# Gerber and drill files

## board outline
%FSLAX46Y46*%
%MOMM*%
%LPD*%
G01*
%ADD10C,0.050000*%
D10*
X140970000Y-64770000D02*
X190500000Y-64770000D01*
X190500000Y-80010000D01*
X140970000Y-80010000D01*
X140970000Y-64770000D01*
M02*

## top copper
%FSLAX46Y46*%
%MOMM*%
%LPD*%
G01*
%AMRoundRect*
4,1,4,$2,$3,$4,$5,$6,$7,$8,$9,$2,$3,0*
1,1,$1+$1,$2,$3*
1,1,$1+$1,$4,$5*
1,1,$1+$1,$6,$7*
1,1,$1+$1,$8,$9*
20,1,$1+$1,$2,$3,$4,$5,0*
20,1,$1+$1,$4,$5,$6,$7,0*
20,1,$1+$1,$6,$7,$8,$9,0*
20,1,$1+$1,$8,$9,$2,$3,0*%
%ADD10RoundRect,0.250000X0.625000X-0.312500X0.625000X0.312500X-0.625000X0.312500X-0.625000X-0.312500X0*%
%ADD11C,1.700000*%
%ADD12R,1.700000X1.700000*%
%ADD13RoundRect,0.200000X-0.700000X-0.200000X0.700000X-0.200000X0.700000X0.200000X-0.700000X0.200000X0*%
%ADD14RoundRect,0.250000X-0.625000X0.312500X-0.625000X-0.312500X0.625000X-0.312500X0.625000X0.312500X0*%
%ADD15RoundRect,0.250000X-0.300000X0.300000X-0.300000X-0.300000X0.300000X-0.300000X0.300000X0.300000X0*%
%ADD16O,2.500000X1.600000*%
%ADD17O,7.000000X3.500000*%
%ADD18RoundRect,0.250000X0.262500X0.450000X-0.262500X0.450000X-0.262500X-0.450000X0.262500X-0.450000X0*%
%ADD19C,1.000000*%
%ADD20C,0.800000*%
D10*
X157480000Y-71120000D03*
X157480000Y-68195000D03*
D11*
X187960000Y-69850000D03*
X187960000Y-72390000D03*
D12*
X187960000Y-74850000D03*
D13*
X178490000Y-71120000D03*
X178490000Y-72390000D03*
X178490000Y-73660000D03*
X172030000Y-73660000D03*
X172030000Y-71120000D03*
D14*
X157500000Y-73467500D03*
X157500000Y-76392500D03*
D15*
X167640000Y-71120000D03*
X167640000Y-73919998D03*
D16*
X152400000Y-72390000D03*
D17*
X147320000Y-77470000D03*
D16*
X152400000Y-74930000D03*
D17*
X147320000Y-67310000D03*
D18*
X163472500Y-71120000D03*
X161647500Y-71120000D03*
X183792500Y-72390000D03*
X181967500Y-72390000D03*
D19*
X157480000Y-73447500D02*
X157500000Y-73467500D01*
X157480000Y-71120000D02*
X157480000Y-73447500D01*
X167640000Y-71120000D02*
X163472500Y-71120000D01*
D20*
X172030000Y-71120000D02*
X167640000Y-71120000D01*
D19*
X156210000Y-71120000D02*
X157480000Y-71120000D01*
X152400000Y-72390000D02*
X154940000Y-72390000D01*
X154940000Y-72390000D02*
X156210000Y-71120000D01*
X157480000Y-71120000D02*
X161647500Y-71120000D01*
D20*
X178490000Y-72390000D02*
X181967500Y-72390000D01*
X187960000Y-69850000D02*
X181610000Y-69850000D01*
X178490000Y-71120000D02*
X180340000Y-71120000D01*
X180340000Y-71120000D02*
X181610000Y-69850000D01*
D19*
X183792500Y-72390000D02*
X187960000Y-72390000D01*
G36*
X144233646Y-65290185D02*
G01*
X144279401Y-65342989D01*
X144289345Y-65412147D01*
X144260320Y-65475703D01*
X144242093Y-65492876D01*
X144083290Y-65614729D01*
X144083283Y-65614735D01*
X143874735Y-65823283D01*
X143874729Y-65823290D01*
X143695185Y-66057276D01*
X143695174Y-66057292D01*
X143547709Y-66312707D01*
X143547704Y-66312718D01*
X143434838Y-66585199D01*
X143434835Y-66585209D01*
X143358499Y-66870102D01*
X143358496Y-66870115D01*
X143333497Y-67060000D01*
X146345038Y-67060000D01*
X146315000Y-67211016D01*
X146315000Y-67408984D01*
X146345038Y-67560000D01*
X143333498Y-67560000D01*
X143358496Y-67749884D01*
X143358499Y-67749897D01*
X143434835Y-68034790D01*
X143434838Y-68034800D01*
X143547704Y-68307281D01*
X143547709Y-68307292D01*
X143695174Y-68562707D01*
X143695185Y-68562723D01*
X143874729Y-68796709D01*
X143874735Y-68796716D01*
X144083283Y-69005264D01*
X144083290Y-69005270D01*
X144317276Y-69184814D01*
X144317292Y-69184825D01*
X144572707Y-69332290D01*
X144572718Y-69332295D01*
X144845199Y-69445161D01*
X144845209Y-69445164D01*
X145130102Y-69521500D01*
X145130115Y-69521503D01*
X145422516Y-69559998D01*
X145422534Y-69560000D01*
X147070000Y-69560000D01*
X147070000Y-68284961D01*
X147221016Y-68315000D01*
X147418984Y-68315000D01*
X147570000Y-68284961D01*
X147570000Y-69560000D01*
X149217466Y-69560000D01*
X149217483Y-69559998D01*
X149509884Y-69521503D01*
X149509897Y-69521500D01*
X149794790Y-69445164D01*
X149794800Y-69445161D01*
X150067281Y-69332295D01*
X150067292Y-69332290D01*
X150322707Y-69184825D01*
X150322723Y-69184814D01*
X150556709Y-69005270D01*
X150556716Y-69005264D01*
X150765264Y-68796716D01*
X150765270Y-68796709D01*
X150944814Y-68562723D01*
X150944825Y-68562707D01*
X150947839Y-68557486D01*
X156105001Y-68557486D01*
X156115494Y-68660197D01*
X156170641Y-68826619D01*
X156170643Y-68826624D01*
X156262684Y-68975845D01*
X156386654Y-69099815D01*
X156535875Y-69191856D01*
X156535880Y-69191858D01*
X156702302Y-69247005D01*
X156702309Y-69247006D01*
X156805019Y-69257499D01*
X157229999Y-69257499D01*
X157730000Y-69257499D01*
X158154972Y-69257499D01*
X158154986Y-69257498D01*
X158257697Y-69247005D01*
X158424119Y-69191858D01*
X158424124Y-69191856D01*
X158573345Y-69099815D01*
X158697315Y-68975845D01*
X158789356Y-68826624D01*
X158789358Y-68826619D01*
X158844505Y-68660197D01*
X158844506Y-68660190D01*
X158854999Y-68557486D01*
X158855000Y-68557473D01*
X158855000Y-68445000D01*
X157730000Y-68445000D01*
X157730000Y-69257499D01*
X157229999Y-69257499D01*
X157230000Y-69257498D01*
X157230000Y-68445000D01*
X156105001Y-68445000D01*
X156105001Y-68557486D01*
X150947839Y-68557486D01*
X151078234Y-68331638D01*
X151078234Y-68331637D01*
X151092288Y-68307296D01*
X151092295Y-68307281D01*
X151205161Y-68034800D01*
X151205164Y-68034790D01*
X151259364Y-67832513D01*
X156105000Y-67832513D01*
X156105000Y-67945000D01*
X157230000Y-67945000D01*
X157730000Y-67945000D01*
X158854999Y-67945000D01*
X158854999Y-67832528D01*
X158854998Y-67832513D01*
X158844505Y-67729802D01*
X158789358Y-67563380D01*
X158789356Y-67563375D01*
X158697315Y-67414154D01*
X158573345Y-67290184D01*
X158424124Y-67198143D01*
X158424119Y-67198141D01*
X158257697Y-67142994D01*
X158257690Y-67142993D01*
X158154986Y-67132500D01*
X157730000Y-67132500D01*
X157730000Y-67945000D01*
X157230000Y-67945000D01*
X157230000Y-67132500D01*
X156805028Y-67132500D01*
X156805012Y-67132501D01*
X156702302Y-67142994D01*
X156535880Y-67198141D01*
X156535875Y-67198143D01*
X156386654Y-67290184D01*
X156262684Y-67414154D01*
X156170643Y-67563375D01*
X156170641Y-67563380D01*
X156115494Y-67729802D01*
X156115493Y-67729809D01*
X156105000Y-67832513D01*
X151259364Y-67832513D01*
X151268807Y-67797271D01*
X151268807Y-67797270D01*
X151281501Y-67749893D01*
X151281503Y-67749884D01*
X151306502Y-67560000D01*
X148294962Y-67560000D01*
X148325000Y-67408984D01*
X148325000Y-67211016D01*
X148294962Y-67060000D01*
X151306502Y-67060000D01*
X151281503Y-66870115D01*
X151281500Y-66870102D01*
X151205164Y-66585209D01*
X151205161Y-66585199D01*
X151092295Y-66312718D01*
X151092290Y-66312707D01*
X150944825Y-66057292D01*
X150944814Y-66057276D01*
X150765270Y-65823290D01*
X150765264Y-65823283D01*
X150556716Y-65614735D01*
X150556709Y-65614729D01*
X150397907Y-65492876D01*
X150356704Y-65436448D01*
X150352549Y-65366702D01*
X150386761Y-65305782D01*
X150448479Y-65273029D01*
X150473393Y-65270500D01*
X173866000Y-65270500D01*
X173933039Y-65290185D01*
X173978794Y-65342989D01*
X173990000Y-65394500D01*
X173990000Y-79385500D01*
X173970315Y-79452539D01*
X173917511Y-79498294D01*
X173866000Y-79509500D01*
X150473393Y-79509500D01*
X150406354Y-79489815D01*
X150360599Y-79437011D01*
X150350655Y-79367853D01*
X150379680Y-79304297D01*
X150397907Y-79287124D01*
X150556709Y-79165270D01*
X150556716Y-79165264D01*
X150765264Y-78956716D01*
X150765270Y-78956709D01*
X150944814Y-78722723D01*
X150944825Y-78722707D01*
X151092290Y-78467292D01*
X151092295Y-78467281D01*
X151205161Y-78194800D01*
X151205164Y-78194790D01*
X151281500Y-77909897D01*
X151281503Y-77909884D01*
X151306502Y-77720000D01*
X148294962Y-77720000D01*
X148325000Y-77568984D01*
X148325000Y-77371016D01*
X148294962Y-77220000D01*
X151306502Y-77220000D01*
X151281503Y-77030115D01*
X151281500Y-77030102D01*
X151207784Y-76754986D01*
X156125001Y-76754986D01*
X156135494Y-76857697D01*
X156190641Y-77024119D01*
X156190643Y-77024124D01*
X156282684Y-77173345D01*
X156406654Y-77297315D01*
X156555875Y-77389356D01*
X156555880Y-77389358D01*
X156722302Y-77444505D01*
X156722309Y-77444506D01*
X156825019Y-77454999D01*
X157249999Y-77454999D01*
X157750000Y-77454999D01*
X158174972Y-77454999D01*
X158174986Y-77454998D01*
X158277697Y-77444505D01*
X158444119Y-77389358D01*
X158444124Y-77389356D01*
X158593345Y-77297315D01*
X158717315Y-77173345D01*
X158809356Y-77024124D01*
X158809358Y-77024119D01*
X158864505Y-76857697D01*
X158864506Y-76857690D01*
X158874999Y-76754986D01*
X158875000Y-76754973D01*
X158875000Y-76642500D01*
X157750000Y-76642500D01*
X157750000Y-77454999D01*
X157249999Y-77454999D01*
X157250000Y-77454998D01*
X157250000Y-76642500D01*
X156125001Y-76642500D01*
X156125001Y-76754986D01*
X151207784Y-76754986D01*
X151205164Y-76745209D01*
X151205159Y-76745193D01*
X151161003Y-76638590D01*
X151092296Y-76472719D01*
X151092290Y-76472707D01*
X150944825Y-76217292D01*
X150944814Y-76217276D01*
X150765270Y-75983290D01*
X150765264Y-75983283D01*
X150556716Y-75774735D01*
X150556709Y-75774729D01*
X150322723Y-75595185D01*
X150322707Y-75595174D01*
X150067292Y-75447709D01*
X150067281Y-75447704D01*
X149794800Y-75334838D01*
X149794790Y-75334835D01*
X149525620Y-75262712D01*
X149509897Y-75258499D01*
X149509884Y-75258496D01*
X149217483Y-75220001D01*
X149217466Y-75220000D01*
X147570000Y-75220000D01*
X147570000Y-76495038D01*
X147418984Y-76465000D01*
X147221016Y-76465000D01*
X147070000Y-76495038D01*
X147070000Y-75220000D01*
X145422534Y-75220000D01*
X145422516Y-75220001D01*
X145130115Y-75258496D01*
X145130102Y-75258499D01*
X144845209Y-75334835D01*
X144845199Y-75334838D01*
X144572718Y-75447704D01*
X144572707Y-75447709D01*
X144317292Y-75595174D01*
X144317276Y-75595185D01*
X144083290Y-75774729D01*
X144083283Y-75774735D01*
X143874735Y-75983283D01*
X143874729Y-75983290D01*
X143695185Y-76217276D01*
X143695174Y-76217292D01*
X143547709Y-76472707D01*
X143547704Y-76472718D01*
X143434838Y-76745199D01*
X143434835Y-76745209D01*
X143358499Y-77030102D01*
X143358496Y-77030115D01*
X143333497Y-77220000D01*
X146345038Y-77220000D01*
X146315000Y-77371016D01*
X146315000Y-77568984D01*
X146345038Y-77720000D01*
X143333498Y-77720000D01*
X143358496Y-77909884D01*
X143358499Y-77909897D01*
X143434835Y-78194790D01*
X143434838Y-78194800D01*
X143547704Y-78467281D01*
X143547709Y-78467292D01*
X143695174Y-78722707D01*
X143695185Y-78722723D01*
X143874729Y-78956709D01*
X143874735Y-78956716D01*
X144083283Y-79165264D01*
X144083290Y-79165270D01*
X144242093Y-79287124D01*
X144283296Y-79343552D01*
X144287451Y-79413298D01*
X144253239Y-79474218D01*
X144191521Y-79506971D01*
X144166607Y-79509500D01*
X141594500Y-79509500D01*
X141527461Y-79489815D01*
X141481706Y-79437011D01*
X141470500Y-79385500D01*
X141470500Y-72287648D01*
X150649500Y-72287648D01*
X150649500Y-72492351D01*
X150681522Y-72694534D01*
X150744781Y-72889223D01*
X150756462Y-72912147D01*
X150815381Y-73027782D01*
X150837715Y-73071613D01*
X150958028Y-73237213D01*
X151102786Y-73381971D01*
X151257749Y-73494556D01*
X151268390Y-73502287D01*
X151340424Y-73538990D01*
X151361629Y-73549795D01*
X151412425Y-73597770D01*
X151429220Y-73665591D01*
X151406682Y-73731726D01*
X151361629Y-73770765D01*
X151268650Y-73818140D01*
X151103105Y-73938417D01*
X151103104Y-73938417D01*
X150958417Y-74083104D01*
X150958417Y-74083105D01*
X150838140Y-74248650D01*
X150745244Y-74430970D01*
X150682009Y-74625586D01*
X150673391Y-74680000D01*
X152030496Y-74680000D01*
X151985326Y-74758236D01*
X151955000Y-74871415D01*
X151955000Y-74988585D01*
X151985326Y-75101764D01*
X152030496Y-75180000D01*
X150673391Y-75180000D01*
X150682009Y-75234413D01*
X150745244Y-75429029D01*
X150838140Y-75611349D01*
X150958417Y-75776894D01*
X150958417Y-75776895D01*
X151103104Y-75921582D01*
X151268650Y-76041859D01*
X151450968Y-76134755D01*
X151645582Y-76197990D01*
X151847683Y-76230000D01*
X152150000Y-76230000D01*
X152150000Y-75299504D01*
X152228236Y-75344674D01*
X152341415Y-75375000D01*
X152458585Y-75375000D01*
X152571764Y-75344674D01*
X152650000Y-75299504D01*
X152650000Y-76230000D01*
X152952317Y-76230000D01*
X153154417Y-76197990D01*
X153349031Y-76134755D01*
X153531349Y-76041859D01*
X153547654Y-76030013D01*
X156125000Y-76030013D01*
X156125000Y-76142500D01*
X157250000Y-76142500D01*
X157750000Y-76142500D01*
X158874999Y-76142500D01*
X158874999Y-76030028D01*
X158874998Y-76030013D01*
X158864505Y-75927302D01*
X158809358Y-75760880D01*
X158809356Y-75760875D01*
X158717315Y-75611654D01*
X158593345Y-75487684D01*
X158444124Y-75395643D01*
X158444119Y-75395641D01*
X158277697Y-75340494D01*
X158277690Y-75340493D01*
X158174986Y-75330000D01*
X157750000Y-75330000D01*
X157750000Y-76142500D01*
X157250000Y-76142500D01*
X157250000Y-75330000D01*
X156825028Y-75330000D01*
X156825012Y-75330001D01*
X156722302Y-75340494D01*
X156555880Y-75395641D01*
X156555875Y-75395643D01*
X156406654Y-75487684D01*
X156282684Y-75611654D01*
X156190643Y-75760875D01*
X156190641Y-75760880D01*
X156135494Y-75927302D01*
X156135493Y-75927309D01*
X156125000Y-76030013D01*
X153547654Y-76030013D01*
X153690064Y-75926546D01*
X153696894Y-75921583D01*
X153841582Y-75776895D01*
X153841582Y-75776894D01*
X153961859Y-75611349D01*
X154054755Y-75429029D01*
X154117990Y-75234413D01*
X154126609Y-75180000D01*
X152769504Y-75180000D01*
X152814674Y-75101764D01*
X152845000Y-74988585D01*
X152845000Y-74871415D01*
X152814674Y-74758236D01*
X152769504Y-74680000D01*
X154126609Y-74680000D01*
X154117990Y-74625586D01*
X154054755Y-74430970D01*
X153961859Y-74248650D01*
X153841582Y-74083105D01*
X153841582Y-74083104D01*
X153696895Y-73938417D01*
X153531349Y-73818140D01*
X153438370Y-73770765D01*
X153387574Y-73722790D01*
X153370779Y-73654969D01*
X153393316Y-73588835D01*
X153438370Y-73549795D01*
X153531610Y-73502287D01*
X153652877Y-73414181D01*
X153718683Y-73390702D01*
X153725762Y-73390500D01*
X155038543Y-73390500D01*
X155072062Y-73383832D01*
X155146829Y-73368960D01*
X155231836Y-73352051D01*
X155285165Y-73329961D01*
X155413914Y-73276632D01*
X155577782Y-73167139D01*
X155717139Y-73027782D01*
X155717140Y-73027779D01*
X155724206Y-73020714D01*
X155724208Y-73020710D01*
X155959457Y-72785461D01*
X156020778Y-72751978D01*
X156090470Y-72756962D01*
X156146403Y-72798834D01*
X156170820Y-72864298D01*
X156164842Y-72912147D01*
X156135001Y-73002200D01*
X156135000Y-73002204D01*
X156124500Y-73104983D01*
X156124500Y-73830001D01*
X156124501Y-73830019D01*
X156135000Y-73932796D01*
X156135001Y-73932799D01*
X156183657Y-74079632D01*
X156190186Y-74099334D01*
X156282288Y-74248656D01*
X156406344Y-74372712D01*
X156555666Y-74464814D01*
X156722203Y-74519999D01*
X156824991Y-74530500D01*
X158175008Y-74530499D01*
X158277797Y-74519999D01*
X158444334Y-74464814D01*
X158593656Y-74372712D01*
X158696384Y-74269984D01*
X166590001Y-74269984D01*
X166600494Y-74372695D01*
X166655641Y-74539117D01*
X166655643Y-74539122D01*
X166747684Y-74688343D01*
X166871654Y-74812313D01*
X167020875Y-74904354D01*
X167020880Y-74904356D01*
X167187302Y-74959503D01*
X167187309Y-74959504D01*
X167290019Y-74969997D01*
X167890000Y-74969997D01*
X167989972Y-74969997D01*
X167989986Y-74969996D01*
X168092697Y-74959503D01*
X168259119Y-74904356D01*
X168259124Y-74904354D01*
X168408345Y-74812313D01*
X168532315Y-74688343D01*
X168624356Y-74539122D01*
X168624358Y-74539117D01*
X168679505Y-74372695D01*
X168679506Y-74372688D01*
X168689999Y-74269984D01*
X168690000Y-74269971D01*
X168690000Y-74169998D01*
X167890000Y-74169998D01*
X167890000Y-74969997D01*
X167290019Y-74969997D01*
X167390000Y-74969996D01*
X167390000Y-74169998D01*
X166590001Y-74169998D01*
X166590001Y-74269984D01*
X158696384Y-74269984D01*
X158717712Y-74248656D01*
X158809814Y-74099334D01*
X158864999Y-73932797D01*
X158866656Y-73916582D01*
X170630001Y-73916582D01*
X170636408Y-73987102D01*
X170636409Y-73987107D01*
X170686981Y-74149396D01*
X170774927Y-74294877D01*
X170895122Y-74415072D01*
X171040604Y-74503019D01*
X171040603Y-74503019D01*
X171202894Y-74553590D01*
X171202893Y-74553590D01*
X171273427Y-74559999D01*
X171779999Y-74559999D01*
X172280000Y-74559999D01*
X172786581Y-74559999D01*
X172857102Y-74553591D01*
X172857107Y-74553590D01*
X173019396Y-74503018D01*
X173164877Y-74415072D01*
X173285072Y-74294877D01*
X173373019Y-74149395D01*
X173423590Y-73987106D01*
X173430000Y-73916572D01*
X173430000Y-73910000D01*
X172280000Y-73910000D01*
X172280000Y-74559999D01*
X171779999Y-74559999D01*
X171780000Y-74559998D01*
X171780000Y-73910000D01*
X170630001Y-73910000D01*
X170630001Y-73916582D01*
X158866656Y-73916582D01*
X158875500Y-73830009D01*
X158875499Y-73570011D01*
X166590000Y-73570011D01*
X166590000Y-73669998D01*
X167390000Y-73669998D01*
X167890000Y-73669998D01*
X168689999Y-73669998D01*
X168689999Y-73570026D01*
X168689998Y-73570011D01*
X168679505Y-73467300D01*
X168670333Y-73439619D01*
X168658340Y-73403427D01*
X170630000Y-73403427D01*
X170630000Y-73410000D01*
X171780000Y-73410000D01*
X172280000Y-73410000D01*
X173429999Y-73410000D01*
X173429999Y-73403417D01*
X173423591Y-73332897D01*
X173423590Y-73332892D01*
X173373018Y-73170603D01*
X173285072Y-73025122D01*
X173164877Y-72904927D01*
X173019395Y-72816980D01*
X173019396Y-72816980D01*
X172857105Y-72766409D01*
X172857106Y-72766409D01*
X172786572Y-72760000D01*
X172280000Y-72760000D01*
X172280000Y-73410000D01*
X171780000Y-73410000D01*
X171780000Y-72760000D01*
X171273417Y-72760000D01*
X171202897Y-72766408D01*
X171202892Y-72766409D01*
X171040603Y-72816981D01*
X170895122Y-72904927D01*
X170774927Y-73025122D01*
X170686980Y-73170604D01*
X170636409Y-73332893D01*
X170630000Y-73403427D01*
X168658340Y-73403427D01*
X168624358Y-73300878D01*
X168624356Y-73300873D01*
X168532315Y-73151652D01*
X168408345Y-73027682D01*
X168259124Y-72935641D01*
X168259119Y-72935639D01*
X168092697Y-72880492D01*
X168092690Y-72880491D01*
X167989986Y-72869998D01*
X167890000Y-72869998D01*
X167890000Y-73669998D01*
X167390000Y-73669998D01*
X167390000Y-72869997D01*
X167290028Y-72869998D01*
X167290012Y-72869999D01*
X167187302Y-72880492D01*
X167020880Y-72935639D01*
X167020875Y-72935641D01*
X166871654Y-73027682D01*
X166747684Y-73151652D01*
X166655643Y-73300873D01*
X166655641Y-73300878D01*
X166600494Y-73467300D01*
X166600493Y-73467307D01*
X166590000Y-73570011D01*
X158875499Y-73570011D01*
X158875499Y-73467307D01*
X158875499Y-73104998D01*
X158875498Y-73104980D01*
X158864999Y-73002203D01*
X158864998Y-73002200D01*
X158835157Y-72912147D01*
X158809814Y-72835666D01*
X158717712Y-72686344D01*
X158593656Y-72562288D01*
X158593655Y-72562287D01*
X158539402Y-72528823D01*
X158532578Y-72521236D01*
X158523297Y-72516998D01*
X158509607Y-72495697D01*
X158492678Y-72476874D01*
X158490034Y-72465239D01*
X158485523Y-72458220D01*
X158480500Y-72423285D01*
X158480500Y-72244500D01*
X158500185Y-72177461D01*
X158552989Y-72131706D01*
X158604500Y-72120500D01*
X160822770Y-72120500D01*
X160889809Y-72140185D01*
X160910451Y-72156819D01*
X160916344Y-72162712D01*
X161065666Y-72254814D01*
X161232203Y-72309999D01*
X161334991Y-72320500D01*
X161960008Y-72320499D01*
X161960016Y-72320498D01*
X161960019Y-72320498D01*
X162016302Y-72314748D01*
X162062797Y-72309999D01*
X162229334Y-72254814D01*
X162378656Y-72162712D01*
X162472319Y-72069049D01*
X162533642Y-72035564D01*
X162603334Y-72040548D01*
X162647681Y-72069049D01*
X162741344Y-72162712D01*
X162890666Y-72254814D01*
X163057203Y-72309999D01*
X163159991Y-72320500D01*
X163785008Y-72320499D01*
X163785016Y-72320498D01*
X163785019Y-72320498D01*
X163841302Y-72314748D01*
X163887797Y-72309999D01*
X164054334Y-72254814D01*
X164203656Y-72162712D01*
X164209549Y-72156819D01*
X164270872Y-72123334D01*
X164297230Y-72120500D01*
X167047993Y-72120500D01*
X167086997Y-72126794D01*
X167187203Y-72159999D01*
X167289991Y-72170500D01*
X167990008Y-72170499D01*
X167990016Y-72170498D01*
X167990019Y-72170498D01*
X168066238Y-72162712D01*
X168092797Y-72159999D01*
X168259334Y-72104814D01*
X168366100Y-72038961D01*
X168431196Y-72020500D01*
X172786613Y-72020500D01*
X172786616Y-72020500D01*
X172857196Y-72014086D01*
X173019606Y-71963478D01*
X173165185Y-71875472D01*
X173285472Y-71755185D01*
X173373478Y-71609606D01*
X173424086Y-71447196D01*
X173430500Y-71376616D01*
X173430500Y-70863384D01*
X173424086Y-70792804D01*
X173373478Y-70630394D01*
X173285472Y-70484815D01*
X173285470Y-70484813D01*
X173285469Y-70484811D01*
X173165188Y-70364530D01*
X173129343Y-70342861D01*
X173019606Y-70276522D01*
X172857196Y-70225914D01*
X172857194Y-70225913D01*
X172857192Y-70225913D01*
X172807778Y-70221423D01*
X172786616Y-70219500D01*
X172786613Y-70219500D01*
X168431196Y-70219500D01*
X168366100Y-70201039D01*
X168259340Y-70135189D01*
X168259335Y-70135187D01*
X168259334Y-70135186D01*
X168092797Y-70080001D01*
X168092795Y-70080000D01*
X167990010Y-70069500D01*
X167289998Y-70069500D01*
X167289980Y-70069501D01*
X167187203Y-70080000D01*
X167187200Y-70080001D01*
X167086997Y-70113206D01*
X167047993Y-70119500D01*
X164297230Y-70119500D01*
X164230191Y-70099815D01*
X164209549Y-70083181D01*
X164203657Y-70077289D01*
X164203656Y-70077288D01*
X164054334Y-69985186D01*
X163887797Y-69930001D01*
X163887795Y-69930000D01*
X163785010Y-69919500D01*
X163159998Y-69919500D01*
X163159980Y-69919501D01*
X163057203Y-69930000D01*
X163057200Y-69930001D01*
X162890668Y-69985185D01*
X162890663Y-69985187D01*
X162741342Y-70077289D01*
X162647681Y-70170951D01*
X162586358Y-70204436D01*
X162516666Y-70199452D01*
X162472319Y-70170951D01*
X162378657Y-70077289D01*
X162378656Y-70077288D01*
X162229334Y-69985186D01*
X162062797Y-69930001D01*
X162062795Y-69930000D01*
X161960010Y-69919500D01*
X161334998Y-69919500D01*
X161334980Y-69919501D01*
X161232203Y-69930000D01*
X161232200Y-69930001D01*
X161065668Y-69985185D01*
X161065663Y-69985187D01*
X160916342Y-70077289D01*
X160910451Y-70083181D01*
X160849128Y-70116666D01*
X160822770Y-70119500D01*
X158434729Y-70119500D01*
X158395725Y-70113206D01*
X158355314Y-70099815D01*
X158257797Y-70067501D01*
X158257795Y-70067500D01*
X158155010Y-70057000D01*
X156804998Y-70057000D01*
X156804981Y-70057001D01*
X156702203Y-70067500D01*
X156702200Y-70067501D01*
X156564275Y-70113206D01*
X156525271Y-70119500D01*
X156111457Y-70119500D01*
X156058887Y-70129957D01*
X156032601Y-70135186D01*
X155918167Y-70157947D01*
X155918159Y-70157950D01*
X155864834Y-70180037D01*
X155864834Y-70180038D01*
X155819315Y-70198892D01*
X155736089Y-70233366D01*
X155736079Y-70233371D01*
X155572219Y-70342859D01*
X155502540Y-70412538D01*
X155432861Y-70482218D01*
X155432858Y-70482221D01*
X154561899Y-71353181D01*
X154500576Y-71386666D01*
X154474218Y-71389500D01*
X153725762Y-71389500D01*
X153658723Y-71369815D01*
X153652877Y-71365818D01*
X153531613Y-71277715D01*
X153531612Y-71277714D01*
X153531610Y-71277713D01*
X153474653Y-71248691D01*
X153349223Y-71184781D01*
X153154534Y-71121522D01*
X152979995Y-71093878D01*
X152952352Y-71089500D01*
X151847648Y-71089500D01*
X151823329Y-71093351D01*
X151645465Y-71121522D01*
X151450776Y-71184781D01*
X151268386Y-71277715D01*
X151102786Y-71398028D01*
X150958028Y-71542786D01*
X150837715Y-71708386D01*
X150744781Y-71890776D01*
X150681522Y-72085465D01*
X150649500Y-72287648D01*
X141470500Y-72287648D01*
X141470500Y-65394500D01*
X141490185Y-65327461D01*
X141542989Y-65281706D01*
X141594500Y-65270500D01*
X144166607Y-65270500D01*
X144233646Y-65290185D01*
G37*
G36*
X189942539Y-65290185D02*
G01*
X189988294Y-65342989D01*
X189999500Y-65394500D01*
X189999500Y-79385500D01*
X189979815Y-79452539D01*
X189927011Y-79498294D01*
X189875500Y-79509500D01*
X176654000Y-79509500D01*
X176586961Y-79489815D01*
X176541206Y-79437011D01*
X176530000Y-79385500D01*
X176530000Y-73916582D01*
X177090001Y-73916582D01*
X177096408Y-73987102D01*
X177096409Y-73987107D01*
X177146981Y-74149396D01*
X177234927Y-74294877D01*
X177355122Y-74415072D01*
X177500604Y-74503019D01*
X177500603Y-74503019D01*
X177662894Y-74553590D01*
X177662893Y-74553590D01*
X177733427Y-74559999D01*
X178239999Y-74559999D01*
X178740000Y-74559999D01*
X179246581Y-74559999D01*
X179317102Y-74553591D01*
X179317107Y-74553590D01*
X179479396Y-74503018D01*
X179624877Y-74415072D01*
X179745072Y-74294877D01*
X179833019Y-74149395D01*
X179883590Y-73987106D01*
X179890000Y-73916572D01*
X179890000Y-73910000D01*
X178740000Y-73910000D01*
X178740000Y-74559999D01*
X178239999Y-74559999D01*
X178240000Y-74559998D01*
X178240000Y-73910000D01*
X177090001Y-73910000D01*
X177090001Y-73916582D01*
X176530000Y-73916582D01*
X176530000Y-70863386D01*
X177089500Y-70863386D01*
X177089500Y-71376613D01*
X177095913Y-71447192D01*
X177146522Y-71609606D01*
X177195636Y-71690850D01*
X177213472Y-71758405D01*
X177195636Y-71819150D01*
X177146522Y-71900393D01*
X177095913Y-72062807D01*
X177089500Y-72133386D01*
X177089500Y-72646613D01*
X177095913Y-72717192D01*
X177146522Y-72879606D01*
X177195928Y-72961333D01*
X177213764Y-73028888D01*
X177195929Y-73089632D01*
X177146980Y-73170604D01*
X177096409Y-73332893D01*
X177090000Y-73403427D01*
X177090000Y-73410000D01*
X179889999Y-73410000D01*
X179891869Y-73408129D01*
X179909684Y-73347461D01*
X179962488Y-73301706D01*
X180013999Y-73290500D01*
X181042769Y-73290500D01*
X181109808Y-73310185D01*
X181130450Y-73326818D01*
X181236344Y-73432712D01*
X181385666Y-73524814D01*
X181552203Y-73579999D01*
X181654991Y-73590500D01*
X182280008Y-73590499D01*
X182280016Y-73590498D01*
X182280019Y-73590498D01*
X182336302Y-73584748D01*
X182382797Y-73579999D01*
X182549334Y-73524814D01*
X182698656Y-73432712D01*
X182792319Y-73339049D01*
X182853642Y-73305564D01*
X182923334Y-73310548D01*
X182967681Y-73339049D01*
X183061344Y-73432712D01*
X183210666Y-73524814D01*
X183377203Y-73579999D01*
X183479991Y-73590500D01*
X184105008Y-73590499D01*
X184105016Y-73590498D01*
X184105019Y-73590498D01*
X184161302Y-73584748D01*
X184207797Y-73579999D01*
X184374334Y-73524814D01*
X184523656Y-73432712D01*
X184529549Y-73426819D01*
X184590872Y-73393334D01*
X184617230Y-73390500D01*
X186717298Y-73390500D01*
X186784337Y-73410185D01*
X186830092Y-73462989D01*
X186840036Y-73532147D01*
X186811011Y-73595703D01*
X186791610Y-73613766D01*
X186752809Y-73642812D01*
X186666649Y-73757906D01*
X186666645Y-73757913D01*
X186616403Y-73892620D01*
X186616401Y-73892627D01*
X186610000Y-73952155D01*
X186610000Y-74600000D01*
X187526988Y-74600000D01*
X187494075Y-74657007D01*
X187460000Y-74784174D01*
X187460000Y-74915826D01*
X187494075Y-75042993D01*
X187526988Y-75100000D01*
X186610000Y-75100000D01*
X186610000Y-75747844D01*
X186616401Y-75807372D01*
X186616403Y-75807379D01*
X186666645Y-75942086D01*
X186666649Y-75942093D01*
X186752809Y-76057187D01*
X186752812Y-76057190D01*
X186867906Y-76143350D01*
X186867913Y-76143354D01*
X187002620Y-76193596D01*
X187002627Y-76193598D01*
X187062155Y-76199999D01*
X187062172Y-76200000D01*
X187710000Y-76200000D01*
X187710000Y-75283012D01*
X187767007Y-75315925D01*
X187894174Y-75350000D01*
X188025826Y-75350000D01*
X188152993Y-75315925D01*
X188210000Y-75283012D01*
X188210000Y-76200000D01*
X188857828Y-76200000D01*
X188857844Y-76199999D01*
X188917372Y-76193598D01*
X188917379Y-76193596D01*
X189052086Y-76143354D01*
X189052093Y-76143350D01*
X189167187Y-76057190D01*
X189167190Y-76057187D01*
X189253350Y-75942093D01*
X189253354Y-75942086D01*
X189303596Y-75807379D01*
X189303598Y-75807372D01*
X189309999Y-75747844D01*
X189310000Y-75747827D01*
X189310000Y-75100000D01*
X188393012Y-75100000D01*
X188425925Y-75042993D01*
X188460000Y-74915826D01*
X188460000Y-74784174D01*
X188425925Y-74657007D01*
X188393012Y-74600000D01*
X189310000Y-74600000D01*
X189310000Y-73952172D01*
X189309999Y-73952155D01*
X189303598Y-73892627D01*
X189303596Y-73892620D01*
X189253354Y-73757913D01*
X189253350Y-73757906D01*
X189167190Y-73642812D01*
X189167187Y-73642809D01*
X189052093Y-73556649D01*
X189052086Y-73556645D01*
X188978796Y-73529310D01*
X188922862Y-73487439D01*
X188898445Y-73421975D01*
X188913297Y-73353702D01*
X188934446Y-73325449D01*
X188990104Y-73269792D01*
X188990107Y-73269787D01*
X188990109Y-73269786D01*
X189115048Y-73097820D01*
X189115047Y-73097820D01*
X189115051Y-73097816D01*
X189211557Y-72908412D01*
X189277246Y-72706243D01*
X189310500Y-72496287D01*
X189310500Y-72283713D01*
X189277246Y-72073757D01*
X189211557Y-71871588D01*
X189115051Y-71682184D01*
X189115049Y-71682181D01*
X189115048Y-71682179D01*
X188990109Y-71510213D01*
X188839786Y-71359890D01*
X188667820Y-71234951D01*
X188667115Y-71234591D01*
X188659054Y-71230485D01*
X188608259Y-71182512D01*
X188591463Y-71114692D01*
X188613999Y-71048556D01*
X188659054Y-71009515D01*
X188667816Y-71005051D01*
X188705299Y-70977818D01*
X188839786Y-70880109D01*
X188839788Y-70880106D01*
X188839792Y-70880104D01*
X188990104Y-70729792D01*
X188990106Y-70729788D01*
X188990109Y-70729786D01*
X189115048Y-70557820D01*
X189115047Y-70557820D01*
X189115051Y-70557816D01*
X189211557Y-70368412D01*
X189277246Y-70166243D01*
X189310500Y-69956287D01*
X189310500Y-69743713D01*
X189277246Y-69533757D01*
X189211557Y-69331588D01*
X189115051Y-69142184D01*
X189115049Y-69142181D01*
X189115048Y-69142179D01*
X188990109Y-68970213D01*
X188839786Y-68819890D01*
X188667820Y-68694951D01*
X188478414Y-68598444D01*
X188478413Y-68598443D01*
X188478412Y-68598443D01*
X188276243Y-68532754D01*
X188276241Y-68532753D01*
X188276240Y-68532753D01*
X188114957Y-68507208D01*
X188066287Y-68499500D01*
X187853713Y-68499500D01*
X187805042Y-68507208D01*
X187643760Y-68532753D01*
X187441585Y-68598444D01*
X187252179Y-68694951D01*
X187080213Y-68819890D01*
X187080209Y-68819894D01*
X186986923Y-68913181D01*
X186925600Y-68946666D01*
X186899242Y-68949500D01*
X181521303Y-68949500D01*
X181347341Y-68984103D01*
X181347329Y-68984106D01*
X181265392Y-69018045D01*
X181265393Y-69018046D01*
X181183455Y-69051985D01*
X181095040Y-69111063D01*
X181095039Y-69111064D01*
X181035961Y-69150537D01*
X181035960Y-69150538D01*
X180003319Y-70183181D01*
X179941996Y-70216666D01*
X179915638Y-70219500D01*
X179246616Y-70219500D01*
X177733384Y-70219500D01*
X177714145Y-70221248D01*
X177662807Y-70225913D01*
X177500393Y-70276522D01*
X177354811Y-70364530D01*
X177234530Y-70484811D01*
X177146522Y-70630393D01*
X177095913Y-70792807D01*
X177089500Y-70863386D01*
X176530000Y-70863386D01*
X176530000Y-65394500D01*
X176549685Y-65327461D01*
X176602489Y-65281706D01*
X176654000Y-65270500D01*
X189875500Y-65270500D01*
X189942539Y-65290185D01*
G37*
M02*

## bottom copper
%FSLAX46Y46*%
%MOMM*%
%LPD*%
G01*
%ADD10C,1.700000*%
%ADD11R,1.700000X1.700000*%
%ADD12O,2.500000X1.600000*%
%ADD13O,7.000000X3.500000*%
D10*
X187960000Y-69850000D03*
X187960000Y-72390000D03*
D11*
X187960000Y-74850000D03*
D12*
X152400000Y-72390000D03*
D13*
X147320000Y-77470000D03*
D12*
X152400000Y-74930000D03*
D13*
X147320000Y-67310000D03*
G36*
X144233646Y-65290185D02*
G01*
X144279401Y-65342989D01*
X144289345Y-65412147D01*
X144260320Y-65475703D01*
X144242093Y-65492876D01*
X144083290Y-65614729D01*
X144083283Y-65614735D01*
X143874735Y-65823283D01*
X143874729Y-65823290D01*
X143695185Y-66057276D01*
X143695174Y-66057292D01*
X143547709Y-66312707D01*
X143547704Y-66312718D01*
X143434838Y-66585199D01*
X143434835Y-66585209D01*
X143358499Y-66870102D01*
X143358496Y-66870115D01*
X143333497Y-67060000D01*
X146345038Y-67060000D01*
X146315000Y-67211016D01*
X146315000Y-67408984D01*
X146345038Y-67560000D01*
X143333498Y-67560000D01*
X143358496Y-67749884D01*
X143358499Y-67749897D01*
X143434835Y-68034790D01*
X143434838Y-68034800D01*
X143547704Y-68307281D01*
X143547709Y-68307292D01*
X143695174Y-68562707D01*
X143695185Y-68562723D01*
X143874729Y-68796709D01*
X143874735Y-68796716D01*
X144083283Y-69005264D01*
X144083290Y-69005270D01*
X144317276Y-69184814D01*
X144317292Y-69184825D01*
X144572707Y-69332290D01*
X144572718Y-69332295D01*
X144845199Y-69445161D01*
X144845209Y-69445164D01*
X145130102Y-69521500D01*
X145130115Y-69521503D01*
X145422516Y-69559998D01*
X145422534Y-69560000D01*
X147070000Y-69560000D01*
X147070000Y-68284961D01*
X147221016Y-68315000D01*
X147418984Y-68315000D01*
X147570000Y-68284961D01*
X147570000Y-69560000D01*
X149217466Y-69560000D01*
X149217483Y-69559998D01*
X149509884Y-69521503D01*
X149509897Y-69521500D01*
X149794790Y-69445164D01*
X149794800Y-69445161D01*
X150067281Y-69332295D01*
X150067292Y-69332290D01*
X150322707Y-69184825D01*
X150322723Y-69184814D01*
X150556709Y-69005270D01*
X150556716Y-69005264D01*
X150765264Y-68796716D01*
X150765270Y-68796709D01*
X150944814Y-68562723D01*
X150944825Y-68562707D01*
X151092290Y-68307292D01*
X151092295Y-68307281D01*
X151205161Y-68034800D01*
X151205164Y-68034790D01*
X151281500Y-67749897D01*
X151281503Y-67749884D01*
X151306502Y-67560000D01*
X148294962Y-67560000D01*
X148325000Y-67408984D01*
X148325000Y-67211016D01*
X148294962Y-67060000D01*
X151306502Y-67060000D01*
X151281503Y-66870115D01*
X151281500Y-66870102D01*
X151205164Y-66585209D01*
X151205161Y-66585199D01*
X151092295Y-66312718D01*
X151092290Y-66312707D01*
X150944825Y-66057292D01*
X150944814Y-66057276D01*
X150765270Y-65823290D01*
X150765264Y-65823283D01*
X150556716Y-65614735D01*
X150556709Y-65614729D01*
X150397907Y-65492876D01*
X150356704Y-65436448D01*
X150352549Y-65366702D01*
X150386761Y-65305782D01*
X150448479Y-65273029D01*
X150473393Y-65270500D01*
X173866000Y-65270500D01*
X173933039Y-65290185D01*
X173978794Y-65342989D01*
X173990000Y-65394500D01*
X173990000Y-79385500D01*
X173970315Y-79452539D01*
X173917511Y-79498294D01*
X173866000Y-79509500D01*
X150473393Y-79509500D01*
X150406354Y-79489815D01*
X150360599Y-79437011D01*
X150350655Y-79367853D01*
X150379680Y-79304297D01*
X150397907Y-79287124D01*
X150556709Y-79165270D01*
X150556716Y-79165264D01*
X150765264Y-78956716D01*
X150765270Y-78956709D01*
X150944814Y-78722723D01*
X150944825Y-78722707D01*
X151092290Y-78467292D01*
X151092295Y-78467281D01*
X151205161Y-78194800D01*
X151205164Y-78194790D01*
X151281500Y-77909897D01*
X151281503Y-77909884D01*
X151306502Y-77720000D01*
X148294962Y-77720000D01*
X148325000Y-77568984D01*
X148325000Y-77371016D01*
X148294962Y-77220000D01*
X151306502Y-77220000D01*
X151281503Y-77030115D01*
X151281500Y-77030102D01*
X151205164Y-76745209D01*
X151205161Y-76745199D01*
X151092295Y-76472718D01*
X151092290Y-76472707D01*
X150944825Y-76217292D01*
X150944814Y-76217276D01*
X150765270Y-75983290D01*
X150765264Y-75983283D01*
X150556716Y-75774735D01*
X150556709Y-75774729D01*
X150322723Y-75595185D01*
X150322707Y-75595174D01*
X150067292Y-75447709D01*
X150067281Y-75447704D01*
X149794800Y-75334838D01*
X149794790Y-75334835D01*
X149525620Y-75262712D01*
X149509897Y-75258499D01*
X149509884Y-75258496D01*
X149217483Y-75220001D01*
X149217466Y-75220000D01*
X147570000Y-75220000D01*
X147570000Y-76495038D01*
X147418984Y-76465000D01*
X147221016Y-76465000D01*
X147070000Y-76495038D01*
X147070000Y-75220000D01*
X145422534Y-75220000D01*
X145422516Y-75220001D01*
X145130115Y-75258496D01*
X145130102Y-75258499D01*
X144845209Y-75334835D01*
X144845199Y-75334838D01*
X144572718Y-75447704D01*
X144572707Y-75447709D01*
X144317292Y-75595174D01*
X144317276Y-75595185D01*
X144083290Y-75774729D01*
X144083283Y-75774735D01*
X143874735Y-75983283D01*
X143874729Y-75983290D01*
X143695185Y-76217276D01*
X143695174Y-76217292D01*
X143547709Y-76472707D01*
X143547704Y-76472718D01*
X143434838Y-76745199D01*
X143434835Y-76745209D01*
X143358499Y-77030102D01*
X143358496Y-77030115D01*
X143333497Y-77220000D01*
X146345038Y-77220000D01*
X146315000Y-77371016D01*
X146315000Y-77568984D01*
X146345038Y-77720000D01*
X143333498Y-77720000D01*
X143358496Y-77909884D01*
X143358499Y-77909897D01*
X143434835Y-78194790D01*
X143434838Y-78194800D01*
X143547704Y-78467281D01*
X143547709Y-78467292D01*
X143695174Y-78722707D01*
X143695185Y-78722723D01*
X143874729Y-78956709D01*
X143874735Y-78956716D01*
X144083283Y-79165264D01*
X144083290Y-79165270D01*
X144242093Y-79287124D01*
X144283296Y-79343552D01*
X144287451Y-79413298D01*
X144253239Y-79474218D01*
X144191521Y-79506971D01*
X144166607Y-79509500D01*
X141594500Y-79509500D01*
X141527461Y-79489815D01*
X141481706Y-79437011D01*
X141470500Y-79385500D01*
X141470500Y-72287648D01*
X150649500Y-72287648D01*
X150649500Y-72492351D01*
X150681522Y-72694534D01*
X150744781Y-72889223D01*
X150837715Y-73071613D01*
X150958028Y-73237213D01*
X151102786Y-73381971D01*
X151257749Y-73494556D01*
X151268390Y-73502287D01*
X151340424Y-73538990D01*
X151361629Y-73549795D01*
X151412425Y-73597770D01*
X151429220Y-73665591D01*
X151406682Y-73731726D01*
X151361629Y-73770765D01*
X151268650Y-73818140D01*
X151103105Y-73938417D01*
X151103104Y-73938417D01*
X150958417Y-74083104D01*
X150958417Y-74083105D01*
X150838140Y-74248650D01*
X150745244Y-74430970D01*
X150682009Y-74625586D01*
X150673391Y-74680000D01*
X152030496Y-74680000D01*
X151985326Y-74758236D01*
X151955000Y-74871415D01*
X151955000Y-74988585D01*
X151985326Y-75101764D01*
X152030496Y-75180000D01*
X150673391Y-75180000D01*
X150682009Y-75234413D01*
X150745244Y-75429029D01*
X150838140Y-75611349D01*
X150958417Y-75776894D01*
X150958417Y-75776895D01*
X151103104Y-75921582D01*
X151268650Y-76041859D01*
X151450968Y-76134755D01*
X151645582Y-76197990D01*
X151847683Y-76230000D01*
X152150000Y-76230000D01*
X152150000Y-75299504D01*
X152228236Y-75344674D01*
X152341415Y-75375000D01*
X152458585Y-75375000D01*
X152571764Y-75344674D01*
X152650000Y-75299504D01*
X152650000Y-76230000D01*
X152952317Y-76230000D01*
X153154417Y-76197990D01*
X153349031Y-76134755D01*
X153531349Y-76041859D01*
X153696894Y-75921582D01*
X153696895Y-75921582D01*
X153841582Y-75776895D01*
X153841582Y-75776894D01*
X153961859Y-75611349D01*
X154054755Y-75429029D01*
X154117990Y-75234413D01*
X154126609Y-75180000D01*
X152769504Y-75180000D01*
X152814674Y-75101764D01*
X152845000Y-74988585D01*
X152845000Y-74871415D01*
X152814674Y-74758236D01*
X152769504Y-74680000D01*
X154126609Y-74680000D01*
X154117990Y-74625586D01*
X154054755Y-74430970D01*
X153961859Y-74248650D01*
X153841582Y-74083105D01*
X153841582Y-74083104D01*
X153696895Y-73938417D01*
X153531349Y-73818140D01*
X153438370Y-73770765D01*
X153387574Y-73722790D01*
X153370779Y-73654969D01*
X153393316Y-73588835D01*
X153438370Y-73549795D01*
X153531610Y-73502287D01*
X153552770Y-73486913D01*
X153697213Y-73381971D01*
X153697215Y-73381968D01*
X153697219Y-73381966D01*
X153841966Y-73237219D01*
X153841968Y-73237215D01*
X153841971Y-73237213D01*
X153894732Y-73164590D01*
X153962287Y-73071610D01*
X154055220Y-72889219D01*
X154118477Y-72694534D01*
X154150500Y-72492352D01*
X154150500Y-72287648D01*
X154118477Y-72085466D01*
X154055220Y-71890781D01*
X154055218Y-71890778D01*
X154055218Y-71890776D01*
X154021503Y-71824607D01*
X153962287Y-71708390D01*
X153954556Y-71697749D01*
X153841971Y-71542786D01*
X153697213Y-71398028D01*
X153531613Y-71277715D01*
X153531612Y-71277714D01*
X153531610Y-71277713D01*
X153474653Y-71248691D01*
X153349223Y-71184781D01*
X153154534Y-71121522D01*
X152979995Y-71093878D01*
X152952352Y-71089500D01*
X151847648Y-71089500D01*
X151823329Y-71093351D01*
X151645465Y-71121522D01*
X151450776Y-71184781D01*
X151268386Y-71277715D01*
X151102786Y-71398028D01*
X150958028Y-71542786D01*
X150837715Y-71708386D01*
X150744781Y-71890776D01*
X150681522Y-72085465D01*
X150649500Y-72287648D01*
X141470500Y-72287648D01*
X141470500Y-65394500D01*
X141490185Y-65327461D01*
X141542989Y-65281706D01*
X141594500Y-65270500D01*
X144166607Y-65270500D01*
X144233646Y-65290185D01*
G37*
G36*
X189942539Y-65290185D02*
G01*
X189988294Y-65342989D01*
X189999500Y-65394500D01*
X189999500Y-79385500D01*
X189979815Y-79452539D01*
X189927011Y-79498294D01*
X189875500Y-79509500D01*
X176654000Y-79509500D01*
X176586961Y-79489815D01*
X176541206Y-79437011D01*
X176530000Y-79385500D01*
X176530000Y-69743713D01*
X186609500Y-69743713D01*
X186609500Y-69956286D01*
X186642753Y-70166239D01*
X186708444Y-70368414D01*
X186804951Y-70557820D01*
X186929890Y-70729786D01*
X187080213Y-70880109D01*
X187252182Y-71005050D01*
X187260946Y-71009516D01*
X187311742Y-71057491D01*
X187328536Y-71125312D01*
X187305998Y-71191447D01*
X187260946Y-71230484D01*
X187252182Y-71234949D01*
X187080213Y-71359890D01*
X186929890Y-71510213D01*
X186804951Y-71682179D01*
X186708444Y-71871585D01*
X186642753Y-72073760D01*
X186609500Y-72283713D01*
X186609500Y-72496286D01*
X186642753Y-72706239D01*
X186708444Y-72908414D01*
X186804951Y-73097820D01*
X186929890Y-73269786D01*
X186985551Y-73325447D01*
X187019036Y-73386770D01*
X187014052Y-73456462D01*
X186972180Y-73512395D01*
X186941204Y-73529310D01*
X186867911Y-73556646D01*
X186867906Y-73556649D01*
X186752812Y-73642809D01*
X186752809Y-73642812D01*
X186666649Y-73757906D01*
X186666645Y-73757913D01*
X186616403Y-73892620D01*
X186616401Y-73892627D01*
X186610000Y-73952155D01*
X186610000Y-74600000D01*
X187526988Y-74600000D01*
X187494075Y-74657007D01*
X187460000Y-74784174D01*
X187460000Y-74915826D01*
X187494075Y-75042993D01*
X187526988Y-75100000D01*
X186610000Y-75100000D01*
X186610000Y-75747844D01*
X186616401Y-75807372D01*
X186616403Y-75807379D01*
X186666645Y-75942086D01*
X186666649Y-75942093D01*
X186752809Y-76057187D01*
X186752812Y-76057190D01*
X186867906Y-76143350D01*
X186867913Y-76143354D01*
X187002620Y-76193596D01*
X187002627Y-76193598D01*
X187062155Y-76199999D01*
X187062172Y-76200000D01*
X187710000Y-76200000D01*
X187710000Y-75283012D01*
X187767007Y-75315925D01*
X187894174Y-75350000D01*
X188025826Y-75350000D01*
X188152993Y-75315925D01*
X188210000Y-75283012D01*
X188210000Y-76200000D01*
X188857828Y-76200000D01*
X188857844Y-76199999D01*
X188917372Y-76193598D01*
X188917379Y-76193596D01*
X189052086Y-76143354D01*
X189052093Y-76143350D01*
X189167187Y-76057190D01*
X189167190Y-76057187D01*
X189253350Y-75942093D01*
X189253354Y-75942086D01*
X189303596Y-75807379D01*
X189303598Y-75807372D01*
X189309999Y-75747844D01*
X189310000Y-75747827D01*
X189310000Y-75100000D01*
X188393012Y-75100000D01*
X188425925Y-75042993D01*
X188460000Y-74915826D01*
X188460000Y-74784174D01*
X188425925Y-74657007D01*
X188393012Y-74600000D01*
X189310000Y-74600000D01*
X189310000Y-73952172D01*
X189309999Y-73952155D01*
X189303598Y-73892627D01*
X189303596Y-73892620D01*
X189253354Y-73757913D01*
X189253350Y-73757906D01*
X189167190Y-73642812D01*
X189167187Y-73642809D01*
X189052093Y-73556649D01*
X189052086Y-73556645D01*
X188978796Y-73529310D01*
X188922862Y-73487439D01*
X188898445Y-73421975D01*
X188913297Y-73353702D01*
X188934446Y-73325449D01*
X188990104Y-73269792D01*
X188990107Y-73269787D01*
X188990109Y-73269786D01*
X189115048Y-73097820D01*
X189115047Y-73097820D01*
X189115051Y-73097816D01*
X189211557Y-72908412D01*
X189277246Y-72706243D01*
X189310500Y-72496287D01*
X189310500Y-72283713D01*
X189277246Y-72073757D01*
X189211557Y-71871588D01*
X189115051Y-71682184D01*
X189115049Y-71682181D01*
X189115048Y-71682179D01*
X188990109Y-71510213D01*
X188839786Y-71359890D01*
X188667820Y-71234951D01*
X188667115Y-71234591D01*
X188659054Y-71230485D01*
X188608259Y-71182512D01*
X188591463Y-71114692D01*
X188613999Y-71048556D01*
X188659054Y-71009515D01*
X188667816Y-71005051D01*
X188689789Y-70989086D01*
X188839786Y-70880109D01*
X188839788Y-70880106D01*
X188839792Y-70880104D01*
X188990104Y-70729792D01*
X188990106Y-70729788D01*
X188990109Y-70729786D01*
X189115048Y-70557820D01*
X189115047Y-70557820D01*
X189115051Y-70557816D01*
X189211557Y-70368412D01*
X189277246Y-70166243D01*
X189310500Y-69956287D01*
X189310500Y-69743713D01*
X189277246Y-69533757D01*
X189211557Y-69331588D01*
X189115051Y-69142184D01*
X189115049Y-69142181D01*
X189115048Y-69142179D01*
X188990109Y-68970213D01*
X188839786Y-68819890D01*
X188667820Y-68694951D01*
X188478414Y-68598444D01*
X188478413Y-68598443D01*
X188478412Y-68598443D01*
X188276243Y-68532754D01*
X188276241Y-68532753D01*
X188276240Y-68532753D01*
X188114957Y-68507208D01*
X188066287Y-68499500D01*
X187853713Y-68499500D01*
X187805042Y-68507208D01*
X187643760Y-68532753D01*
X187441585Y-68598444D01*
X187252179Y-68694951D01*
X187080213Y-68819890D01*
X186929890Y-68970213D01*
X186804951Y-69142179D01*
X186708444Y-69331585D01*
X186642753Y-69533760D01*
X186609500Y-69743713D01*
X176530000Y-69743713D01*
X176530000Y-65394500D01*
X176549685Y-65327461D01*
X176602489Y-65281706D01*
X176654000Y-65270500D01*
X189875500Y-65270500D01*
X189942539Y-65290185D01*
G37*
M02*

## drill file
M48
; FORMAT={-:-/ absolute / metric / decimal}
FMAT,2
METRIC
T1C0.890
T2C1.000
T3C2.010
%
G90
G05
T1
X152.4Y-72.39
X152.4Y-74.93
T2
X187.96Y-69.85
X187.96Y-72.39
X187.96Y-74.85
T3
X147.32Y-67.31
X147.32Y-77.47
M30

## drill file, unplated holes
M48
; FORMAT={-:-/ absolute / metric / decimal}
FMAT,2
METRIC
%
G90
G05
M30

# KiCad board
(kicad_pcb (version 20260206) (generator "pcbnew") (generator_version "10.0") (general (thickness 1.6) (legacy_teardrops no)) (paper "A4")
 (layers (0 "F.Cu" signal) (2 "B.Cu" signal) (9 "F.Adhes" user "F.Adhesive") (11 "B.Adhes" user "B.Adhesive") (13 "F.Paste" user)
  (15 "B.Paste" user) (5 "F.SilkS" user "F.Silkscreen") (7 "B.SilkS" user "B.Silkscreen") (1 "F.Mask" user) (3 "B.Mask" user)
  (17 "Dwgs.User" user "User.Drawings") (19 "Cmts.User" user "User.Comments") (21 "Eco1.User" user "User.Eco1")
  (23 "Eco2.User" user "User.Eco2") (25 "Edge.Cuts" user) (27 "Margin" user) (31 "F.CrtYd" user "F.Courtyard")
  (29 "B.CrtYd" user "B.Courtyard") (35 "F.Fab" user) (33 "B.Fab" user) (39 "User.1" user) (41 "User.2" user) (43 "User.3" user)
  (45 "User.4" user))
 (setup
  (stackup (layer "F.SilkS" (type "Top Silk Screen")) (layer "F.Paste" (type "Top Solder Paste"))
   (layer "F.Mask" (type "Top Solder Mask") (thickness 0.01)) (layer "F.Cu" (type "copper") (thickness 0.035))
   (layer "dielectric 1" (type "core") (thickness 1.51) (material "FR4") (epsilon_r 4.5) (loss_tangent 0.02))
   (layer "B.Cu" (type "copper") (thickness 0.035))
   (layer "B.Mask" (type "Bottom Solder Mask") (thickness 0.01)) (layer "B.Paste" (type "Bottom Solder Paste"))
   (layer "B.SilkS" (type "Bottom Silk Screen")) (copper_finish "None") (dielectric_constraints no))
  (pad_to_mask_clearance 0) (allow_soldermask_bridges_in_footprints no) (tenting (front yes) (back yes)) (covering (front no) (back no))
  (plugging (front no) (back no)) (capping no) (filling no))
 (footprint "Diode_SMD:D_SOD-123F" (layer "F.Cu") (at 167.64 72.519999 -90)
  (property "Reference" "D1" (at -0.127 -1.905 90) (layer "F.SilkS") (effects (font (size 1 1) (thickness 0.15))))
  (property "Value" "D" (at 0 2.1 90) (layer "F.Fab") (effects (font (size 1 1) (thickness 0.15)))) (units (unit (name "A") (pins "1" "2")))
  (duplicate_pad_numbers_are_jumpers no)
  (pad "1" smd roundrect (at -1.399999 0 270) (size 1.1 1.1) (layers "F.Cu" "F.Mask" "F.Paste") (roundrect_rratio 0.2272727273)
   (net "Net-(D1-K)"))
  (pad "2" smd roundrect (at 1.399999 0 270) (size 1.1 1.1) (layers "F.Cu" "F.Mask" "F.Paste") (roundrect_rratio 0.2272727273) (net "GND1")))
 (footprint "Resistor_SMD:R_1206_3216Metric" (layer "F.Cu") (at 157.48 69.6575 90)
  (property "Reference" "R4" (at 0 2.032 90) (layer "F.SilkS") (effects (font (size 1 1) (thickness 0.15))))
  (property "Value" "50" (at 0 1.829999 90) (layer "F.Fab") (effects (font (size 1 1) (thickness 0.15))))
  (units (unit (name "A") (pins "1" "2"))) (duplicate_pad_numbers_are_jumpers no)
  (pad "1" smd roundrect (at -1.4625 0 90) (size 1.125 1.75) (layers "F.Cu" "F.Mask" "F.Paste") (roundrect_rratio 0.222222)
   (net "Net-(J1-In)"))
  (pad "2" smd roundrect (at 1.4625 0 90) (size 1.125 1.75) (layers "F.Cu" "F.Mask" "F.Paste") (roundrect_rratio 0.222222) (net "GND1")))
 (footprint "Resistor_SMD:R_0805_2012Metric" (layer "F.Cu") (at 162.56 71.12 180)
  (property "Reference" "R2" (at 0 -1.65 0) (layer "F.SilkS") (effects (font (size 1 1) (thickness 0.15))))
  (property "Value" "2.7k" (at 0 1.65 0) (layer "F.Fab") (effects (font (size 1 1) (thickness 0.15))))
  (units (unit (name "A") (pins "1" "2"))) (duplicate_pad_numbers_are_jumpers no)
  (pad "1" smd roundrect (at -0.9125 0 180) (size 1.025 1.4) (layers "F.Cu" "F.Mask" "F.Paste") (roundrect_rratio 0.243902)
   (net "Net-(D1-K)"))
  (pad "2" smd roundrect (at 0.9125 0 180) (size 1.025 1.4) (layers "F.Cu" "F.Mask" "F.Paste") (roundrect_rratio 0.243902)
   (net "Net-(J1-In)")))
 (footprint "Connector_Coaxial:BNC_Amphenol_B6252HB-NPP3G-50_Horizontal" (layer "F.Cu") (at 152.4 72.39 90)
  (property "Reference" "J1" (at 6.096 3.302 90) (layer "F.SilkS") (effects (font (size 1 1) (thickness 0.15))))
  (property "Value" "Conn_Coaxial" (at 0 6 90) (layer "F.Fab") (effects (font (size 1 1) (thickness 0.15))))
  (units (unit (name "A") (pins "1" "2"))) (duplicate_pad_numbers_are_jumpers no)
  (pad "1" thru_hole oval (at 0 0 90) (size 1.6 2.5) (drill 0.89) (layers "*.Cu" "*.Mask") (remove_unused_layers no) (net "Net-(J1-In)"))
  (pad "2" thru_hole oval (at -5.08 -5.08 90) (size 3.5 7) (drill 2.01) (layers "*.Cu" "*.Mask") (remove_unused_layers no) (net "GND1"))
  (pad "2" thru_hole oval (at -2.54 0 90) (size 1.6 2.5) (drill 0.89) (layers "*.Cu" "*.Mask") (remove_unused_layers no) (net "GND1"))
  (pad "2" thru_hole oval (at 5.08 -5.08 90) (size 3.5 7) (drill 2.01) (layers "*.Cu" "*.Mask") (remove_unused_layers no) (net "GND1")))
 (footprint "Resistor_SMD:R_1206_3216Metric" (layer "F.Cu") (at 157.5 74.93 -90)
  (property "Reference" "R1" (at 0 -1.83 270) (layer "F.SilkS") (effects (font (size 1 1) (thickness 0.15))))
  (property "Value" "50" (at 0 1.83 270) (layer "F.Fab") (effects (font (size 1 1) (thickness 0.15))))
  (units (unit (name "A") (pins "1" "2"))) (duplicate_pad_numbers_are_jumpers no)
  (pad "1" smd roundrect (at -1.4625 0 270) (size 1.125 1.75) (layers "F.Cu" "F.Mask" "F.Paste") (roundrect_rratio 0.222222)
   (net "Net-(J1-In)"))
  (pad "2" smd roundrect (at 1.4625 0 270) (size 1.125 1.75) (layers "F.Cu" "F.Mask" "F.Paste") (roundrect_rratio 0.222222) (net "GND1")))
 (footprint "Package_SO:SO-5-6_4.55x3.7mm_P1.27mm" (layer "F.Cu") (at 175.26 72.39)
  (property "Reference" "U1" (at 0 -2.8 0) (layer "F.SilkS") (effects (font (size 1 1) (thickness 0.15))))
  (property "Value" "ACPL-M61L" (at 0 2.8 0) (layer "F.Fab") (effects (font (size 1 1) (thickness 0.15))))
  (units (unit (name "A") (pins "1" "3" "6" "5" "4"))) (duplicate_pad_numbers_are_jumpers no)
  (pad "1" smd roundrect (at -3.23 -1.27) (size 1.8 0.8) (layers "F.Cu" "F.Mask" "F.Paste") (roundrect_rratio 0.25) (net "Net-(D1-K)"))
  (pad "3" smd roundrect (at -3.23 1.27) (size 1.8 0.8) (layers "F.Cu" "F.Mask" "F.Paste") (roundrect_rratio 0.25) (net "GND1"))
  (pad "4" smd roundrect (at 3.23 1.27) (size 1.8 0.8) (layers "F.Cu" "F.Mask" "F.Paste") (roundrect_rratio 0.25) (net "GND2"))
  (pad "5" smd roundrect (at 3.23 0) (size 1.8 0.8) (layers "F.Cu" "F.Mask" "F.Paste") (roundrect_rratio 0.25) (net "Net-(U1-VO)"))
  (pad "6" smd roundrect (at 3.23 -1.27) (size 1.8 0.8) (layers "F.Cu" "F.Mask" "F.Paste") (roundrect_rratio 0.25) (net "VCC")))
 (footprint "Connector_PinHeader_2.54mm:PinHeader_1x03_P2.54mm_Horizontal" (layer "F.Cu") (at 187.96 69.85)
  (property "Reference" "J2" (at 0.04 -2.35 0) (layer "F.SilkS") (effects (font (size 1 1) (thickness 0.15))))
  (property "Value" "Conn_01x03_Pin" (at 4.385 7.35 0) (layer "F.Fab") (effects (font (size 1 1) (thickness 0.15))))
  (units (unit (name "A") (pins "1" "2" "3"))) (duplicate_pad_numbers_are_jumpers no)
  (pad "1" thru_hole rect (at 0 5) (size 1.7 1.7) (drill 1) (layers "*.Cu" "*.Mask") (remove_unused_layers no) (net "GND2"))
  (pad "2" thru_hole circle (at 0 2.54) (size 1.7 1.7) (drill 1) (layers "*.Cu" "*.Mask") (remove_unused_layers no) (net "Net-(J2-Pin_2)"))
  (pad "3" thru_hole circle (at 0 0) (size 1.7 1.7) (drill 1) (layers "*.Cu" "*.Mask") (remove_unused_layers no) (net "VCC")))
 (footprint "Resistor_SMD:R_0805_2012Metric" (layer "F.Cu") (at 182.88 72.39 180)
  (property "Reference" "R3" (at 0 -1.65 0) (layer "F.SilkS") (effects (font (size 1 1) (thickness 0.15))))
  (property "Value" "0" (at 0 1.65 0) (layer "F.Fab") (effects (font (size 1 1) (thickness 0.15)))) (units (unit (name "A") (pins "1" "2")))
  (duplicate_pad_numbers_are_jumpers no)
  (pad "1" smd roundrect (at -0.9125 0 180) (size 1.025 1.4) (layers "F.Cu" "F.Mask" "F.Paste") (roundrect_rratio 0.243902)
   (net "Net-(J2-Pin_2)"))
  (pad "2" smd roundrect (at 0.9125 0 180) (size 1.025 1.4) (layers "F.Cu" "F.Mask" "F.Paste") (roundrect_rratio 0.243902)
   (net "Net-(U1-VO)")))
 (gr_rect (start 140.97 64.77) (end 190.5 80.01) (stroke (width 0.05) (type default)) (fill no) (layer "Edge.Cuts"))
 (segment (start 167.64 71.12) (end 163.4725 71.12) (width 1) (layer "F.Cu") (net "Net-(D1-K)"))
 (segment (start 172.03 71.12) (end 167.64 71.12) (width 0.8) (layer "F.Cu") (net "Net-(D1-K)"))
 (segment (start 156.21 71.12) (end 157.48 71.12) (width 1) (layer "F.Cu") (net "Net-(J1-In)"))
 (segment (start 152.4 72.39) (end 154.94 72.39) (width 1) (layer "F.Cu") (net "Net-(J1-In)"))
 (segment (start 154.94 72.39) (end 156.21 71.12) (width 1) (layer "F.Cu") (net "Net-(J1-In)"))
 (segment (start 157.48 73.4475) (end 157.5 73.4675) (width 1) (layer "F.Cu") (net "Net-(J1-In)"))
 (segment (start 157.48 71.12) (end 161.6475 71.12) (width 1) (layer "F.Cu") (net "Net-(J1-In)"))
 (segment (start 157.48 71.12) (end 157.48 73.4475) (width 1) (layer "F.Cu") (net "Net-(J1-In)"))
 (segment (start 178.49 72.39) (end 181.9675 72.39) (width 0.8) (layer "F.Cu") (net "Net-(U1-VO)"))
 (segment (start 187.96 69.85) (end 181.61 69.85) (width 0.8) (layer "F.Cu") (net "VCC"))
 (segment (start 178.49 71.12) (end 180.34 71.12) (width 0.8) (layer "F.Cu") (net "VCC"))
 (segment (start 180.34 71.12) (end 181.61 69.85) (width 0.8) (layer "F.Cu") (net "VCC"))
 (segment (start 183.7925 72.39) (end 187.96 72.39) (width 1) (layer "F.Cu") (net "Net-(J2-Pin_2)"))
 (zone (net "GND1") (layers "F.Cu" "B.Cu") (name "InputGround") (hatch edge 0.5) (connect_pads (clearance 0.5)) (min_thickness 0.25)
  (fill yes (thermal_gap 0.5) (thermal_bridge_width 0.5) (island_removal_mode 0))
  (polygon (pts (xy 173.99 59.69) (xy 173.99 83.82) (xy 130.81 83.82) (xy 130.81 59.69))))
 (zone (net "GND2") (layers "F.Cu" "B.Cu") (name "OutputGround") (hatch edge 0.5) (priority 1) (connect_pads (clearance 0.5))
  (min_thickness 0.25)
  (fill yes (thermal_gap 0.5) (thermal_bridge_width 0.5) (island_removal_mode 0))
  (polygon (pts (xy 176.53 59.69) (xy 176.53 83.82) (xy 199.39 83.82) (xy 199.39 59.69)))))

